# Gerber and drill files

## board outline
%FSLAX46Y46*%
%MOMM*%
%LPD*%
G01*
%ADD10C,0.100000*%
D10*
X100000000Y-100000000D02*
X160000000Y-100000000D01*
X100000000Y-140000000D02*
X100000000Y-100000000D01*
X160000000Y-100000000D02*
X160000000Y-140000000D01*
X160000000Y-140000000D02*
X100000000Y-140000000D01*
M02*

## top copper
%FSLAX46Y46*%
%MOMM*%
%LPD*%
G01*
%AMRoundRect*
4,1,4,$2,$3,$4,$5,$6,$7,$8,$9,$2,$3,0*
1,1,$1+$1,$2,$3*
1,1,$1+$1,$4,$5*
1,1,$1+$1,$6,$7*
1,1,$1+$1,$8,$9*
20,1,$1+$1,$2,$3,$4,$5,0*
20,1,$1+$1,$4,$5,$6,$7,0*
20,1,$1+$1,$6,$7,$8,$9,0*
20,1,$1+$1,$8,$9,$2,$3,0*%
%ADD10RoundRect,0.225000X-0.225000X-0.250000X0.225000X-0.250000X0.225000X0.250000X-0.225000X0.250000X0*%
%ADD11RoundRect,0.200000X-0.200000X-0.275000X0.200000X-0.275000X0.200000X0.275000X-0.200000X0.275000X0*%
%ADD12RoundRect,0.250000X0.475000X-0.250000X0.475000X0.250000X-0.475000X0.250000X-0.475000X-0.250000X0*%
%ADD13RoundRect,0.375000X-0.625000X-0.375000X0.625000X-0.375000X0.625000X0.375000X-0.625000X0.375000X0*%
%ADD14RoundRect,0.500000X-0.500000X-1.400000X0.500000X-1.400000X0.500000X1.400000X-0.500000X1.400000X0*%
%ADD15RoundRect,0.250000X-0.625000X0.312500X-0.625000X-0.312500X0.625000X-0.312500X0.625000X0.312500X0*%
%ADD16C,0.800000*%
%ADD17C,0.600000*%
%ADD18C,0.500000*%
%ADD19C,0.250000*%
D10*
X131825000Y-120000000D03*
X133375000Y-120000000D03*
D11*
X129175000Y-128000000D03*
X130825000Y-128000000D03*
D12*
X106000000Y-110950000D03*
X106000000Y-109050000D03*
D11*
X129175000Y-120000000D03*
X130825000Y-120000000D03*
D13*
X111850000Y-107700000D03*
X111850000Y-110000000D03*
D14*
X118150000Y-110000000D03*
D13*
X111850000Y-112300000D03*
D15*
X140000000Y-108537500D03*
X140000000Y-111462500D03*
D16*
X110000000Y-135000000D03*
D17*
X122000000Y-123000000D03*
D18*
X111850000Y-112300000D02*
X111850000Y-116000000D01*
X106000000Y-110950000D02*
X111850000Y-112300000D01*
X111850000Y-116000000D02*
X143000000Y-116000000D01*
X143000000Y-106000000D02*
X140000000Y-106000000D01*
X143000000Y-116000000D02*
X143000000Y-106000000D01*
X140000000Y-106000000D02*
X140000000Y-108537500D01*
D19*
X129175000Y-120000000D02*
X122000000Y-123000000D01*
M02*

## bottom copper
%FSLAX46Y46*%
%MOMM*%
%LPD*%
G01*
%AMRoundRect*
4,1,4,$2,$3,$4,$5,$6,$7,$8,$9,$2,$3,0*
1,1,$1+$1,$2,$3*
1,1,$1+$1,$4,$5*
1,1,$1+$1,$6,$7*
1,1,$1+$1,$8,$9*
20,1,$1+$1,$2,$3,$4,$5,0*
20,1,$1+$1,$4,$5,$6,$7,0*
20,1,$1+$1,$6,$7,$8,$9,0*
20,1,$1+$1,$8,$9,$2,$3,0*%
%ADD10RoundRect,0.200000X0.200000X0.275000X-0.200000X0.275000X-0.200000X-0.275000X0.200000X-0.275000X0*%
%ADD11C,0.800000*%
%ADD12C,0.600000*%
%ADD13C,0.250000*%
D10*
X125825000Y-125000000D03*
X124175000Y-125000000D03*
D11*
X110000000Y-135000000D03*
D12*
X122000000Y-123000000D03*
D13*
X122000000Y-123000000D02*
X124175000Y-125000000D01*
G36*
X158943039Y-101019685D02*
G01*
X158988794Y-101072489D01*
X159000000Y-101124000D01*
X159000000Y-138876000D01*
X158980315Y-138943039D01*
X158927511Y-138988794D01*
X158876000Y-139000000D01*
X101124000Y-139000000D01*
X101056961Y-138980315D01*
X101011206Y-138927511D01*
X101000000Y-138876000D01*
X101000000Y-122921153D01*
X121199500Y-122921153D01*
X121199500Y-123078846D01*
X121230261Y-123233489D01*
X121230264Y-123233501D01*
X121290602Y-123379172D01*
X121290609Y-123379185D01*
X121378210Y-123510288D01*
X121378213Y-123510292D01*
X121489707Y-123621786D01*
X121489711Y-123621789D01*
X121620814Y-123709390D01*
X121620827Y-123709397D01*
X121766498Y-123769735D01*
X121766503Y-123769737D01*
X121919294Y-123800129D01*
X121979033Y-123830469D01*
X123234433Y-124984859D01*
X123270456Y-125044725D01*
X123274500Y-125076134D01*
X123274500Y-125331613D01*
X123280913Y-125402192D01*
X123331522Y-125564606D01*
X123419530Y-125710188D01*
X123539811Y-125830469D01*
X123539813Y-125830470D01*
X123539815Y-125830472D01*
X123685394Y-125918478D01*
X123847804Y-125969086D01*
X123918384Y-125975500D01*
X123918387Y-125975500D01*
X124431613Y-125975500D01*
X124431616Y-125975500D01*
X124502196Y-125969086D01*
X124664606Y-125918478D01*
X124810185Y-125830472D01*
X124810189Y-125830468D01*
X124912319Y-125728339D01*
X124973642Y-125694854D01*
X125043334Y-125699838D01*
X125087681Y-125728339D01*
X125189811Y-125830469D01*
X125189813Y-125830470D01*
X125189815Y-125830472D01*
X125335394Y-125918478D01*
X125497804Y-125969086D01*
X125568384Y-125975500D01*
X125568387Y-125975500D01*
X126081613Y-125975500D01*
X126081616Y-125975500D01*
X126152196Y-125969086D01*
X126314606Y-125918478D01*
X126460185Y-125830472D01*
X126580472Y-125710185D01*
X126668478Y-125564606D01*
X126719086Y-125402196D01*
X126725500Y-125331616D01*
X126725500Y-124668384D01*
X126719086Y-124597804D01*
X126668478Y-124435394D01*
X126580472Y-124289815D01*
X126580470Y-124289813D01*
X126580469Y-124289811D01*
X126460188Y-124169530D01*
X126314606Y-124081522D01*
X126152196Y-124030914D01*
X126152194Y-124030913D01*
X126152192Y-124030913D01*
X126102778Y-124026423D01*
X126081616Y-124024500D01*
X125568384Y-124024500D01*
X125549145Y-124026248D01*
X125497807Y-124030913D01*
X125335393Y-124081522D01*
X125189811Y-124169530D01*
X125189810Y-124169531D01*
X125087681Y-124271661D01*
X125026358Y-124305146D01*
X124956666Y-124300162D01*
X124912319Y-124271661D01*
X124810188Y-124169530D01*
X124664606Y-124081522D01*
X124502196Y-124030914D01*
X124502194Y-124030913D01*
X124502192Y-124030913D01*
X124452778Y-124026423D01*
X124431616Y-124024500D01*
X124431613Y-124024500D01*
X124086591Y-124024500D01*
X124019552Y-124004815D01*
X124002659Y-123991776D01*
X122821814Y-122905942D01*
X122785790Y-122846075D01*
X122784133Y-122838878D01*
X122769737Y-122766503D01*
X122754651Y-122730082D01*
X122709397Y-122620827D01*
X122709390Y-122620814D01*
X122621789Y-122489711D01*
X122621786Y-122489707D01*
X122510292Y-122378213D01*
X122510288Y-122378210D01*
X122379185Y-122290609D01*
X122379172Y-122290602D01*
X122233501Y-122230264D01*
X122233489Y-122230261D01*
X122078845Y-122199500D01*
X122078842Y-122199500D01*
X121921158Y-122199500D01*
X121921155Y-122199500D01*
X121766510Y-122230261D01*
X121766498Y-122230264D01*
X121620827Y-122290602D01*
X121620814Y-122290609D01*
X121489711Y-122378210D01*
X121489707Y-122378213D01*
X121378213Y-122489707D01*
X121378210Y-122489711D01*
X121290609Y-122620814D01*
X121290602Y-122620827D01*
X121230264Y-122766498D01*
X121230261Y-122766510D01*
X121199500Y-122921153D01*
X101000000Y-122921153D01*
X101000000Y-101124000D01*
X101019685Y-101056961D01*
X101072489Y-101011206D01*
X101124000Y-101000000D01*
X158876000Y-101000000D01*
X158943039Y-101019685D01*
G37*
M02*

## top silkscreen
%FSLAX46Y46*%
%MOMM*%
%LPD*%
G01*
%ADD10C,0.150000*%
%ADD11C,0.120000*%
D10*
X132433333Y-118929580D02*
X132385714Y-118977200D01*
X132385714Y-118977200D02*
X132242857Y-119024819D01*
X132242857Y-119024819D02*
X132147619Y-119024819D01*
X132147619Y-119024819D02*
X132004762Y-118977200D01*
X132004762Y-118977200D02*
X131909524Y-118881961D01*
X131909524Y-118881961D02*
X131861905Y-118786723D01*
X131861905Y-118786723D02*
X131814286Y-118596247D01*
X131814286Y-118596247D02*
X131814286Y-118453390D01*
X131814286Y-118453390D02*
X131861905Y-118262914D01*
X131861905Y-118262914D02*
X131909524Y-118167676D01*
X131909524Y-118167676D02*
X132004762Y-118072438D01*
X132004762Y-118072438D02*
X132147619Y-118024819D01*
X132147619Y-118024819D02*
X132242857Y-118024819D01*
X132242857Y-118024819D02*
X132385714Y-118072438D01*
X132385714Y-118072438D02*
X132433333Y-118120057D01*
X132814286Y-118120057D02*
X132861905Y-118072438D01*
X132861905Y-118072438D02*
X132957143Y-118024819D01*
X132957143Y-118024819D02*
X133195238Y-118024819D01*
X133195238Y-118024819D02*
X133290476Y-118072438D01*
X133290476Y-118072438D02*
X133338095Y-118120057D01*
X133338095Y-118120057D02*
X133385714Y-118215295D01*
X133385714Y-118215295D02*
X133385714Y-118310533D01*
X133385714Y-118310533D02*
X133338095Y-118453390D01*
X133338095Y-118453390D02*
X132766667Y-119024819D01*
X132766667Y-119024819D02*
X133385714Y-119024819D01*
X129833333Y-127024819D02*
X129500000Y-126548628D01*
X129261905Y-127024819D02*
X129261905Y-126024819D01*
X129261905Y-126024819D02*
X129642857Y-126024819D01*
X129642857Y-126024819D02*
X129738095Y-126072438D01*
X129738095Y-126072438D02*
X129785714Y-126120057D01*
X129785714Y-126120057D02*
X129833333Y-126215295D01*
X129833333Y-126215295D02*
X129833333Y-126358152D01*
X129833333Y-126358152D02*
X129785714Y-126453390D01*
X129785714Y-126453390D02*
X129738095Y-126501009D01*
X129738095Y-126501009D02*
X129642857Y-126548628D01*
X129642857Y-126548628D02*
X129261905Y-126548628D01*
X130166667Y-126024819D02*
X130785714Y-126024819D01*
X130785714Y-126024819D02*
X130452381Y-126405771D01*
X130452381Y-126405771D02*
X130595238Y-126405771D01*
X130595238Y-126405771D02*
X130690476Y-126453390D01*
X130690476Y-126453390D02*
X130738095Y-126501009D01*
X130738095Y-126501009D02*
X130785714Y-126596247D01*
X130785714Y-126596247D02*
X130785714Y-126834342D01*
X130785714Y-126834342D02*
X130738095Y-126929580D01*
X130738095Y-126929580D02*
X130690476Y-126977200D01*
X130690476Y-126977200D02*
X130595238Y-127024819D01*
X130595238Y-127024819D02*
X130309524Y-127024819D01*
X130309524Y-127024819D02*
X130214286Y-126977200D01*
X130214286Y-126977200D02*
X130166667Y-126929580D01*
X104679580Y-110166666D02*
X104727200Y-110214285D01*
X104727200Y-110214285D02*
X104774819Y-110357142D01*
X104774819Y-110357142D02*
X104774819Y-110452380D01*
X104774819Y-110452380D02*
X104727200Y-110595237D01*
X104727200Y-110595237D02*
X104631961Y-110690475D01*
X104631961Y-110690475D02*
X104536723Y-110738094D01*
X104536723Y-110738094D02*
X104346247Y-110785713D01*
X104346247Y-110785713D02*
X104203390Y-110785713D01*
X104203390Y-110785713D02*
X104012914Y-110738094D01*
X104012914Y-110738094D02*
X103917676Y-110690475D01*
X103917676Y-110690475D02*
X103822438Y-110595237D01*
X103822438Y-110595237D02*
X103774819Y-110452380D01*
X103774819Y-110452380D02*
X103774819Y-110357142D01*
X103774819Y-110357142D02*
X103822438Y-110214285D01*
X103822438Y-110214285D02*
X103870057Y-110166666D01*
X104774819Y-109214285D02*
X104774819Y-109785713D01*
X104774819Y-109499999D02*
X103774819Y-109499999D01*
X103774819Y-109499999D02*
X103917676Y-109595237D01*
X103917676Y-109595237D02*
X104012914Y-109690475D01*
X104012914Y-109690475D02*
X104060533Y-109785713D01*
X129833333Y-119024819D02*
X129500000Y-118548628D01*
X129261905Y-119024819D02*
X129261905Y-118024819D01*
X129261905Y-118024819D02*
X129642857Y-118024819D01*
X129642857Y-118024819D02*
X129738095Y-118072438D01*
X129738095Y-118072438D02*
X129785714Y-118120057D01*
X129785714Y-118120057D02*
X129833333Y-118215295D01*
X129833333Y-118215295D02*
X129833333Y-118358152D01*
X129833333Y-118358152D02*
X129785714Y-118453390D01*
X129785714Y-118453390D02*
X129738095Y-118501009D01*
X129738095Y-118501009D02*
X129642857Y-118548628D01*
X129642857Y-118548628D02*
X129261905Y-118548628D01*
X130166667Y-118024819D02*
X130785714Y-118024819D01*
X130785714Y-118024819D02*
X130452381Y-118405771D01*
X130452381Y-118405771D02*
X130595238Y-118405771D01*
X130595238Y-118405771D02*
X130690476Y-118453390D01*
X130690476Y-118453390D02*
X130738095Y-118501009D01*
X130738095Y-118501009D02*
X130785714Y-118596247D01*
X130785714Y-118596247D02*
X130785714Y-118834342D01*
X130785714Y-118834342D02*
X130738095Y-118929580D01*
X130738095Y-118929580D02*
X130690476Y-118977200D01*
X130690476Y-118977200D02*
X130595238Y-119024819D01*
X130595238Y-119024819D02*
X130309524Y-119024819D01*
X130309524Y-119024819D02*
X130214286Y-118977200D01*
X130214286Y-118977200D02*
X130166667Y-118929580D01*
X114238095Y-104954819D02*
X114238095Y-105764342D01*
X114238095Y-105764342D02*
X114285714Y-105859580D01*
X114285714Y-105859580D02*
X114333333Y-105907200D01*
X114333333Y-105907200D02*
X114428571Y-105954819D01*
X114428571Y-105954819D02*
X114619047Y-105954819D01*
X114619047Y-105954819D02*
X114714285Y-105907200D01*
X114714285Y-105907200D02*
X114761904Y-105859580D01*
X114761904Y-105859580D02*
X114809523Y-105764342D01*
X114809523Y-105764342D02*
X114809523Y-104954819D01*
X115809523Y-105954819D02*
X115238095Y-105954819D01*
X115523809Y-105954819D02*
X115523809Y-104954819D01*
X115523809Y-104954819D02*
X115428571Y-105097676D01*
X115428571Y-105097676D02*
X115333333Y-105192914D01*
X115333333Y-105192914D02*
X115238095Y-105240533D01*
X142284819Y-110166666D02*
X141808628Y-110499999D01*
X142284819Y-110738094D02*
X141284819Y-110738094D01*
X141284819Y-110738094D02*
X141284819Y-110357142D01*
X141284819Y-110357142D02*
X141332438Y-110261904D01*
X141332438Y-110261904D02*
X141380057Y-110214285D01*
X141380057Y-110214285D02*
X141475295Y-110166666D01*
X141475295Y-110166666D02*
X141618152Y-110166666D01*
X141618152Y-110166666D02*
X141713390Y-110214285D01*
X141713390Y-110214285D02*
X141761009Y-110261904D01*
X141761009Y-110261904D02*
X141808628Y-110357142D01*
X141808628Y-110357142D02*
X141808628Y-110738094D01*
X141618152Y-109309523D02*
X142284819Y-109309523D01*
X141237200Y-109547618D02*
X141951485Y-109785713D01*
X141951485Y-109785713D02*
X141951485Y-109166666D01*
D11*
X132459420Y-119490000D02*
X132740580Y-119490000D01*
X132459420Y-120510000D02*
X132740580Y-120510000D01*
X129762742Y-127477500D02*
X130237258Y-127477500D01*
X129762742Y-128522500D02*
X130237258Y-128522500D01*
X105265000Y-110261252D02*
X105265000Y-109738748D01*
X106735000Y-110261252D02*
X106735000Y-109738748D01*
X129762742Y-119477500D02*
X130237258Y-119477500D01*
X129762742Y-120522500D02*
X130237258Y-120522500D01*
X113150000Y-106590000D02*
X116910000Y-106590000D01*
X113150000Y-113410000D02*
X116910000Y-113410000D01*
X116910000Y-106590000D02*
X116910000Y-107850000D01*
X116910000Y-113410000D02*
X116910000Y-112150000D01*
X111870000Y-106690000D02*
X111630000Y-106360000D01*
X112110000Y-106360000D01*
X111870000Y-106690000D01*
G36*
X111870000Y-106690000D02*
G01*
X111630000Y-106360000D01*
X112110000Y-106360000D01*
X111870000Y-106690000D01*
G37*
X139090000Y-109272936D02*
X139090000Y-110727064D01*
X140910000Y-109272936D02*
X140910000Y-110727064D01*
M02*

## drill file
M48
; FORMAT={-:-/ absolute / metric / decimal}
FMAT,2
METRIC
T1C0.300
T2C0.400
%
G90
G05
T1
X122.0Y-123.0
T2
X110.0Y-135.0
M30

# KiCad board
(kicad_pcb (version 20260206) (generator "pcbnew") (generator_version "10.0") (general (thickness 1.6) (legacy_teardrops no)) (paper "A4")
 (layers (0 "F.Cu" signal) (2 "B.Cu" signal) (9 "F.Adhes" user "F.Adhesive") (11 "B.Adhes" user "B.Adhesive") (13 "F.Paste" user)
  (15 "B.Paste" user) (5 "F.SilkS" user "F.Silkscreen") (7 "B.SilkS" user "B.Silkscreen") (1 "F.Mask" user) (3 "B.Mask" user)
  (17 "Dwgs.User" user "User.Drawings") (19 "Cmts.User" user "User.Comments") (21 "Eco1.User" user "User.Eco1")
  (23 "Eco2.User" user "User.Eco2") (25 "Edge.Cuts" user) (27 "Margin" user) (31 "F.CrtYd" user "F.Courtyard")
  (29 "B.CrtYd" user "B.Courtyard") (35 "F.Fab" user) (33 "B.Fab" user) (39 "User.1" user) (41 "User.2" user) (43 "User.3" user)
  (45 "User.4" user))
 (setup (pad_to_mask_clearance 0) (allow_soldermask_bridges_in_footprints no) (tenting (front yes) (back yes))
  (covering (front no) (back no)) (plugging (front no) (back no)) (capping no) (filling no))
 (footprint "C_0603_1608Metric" (layer "F.Cu") (at 132.6 120)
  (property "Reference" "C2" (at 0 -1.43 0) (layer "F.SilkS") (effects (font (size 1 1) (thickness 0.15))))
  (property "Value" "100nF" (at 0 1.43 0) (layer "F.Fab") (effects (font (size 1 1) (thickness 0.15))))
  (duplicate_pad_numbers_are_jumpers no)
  (fp_line (start -0.14058 -0.51) (end 0.14058 -0.51) (stroke (width 0.12) (type solid)) (layer "F.SilkS"))
  (fp_line (start -0.14058 0.51) (end 0.14058 0.51) (stroke (width 0.12) (type solid)) (layer "F.SilkS"))
  (pad "1" smd roundrect (at -0.775 0) (size 0.9 0.95) (layers "F.Cu" "F.Mask" "F.Paste") (roundrect_rratio 0.25) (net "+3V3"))
  (pad "2" smd roundrect (at 0.775 0) (size 0.9 0.95) (layers "F.Cu" "F.Mask" "F.Paste") (roundrect_rratio 0.25) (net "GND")))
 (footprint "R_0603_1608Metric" (layer "F.Cu") (at 130 128)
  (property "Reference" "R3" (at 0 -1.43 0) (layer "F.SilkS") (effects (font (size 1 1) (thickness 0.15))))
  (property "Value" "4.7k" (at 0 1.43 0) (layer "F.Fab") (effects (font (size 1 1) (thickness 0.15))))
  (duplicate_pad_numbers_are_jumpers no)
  (fp_line (start -0.237258 -0.5225) (end 0.237258 -0.5225) (stroke (width 0.12) (type solid)) (layer "F.SilkS"))
  (fp_line (start -0.237258 0.5225) (end 0.237258 0.5225) (stroke (width 0.12) (type solid)) (layer "F.SilkS"))
  (pad "1" smd roundrect (at -0.825 0) (size 0.8 0.95) (layers "F.Cu" "F.Mask" "F.Paste") (roundrect_rratio 0.25) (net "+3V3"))
  (pad "2" smd roundrect (at 0.825 0) (size 0.8 0.95) (layers "F.Cu" "F.Mask" "F.Paste") (roundrect_rratio 0.25) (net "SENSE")))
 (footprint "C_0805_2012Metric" (layer "F.Cu") (at 106 110 90)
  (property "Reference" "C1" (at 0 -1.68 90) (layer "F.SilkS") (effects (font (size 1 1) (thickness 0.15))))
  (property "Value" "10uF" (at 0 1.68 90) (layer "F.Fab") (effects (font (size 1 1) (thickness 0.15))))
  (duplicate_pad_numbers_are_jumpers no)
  (fp_line (start -0.261252 -0.735) (end 0.261252 -0.735) (stroke (width 0.12) (type solid)) (layer "F.SilkS"))
  (fp_line (start -0.261252 0.735) (end 0.261252 0.735) (stroke (width 0.12) (type solid)) (layer "F.SilkS"))
  (pad "1" smd roundrect (at -0.95 0 90) (size 1 1.45) (layers "F.Cu" "F.Mask" "F.Paste") (roundrect_rratio 0.25) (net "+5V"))
  (pad "2" smd roundrect (at 0.95 0 90) (size 1 1.45) (layers "F.Cu" "F.Mask" "F.Paste") (roundrect_rratio 0.25) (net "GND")))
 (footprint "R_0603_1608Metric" (layer "F.Cu") (at 130 120)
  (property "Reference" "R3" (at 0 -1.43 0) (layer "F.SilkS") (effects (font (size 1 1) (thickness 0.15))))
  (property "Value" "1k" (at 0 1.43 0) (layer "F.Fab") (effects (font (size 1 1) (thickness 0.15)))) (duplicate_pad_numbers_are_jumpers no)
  (fp_line (start -0.237258 -0.5225) (end 0.237258 -0.5225) (stroke (width 0.12) (type solid)) (layer "F.SilkS"))
  (fp_line (start -0.237258 0.5225) (end 0.237258 0.5225) (stroke (width 0.12) (type solid)) (layer "F.SilkS"))
  (pad "1" smd roundrect (at -0.825 0) (size 0.8 0.95) (layers "F.Cu" "F.Mask" "F.Paste") (roundrect_rratio 0.25) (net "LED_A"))
  (pad "2" smd roundrect (at 0.825 0) (size 0.8 0.95) (layers "F.Cu" "F.Mask" "F.Paste") (roundrect_rratio 0.25) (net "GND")))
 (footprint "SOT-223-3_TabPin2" (layer "F.Cu") (at 115 110)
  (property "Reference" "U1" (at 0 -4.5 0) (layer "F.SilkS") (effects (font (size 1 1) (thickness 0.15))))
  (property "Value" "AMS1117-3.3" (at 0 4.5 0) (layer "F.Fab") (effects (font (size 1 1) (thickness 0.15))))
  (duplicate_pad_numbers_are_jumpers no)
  (fp_line (start -1.85 -3.41) (end 1.91 -3.41) (stroke (width 0.12) (type solid)) (layer "F.SilkS"))
  (fp_line (start -1.85 3.41) (end 1.91 3.41) (stroke (width 0.12) (type solid)) (layer "F.SilkS"))
  (fp_line (start 1.91 -3.41) (end 1.91 -2.15) (stroke (width 0.12) (type solid)) (layer "F.SilkS"))
  (fp_line (start 1.91 3.41) (end 1.91 2.15) (stroke (width 0.12) (type solid)) (layer "F.SilkS"))
  (fp_poly
   (pts (xy -3.13 -3.31) (xy -3.37 -3.64) (xy -2.89 -3.64) (xy -3.13 -3.31)) (stroke (width 0.12) (type solid)) (fill yes) (layer "F.SilkS"))
  (pad "1" smd roundrect (at -3.15 -2.3) (size 2 1.5) (layers "F.Cu" "F.Mask" "F.Paste") (roundrect_rratio 0.25) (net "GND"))
  (pad "2" smd roundrect (at -3.15 0) (size 2 1.5) (layers "F.Cu" "F.Mask" "F.Paste") (roundrect_rratio 0.25) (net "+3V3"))
  (pad "2" smd roundrect (at 3.15 0) (size 2 3.8) (layers "F.Cu" "F.Mask" "F.Paste") (roundrect_rratio 0.25) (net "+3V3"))
  (pad "3" smd roundrect (at -3.15 2.3) (size 2 1.5) (layers "F.Cu" "F.Mask" "F.Paste") (roundrect_rratio 0.25) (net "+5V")))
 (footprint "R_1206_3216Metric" (layer "F.Cu") (at 140 110 -90)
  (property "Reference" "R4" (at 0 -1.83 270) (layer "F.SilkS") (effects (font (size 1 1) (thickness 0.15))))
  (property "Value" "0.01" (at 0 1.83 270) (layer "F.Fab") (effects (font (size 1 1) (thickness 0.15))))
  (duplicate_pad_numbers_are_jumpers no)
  (fp_line (start -0.727064 0.91) (end 0.727064 0.91) (stroke (width 0.12) (type solid)) (layer "F.SilkS"))
  (fp_line (start -0.727064 -0.91) (end 0.727064 -0.91) (stroke (width 0.12) (type solid)) (layer "F.SilkS"))
  (pad "1" smd roundrect (at -1.4625 0 270) (size 1.125 1.75) (layers "F.Cu" "F.Mask" "F.Paste") (roundrect_rratio 0.222222) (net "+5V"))
  (pad "2" smd roundrect (at 1.4625 0 270) (size 1.125 1.75) (layers "F.Cu" "F.Mask" "F.Paste") (roundrect_rratio 0.222222) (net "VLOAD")))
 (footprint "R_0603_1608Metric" (layer "B.Cu") (at 125 125 180)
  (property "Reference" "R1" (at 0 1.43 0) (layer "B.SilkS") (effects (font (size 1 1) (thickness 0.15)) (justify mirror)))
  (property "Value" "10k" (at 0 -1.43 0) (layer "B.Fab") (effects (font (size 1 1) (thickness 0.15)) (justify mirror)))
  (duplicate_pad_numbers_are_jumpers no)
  (pad "1" smd roundrect (at -0.825 0 180) (size 0.8 0.95) (layers "B.Cu" "B.Mask" "B.Paste") (roundrect_rratio 0.25) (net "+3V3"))
  (pad "2" smd roundrect (at 0.825 0 180) (size 0.8 0.95) (layers "B.Cu" "B.Mask" "B.Paste") (roundrect_rratio 0.25) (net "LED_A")))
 (gr_line (start 100 100) (end 160 100) (stroke (width 0.1) (type default)) (layer "Edge.Cuts"))
 (gr_line (start 100 140) (end 100 100) (stroke (width 0.1) (type default)) (layer "Edge.Cuts"))
 (gr_line (start 160 100) (end 160 140) (stroke (width 0.1) (type default)) (layer "Edge.Cuts"))
 (gr_line (start 160 140) (end 100 140) (stroke (width 0.1) (type default)) (layer "Edge.Cuts"))
 (via (at 110 135) (size 0.8) (drill 0.4) (layers "F.Cu" "B.Cu") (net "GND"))
 (segment (start 111.85 112.3) (end 111.85 116) (width 0.5) (layer "F.Cu") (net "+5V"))
 (segment (start 106 110.95) (end 111.85 112.3) (width 0.5) (layer "F.Cu") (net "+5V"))
 (segment (start 111.85 116) (end 143 116) (width 0.5) (layer "F.Cu") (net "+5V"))
 (segment (start 143 106) (end 140 106) (width 0.5) (layer "F.Cu") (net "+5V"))
 (segment (start 143 116) (end 143 106) (width 0.5) (layer "F.Cu") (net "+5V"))
 (segment (start 140 106) (end 140 108.5375) (width 0.5) (layer "F.Cu") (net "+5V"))
 (segment (start 129.175 120) (end 122 123) (width 0.25) (layer "F.Cu") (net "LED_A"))
 (via (at 122 123) (size 0.6) (drill 0.3) (layers "F.Cu" "B.Cu") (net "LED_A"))
 (segment (start 122 123) (end 124.175 125) (width 0.25) (layer "B.Cu") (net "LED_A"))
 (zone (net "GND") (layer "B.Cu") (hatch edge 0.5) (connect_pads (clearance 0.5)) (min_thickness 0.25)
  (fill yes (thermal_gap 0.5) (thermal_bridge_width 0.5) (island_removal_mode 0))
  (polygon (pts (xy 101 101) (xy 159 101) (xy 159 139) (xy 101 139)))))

